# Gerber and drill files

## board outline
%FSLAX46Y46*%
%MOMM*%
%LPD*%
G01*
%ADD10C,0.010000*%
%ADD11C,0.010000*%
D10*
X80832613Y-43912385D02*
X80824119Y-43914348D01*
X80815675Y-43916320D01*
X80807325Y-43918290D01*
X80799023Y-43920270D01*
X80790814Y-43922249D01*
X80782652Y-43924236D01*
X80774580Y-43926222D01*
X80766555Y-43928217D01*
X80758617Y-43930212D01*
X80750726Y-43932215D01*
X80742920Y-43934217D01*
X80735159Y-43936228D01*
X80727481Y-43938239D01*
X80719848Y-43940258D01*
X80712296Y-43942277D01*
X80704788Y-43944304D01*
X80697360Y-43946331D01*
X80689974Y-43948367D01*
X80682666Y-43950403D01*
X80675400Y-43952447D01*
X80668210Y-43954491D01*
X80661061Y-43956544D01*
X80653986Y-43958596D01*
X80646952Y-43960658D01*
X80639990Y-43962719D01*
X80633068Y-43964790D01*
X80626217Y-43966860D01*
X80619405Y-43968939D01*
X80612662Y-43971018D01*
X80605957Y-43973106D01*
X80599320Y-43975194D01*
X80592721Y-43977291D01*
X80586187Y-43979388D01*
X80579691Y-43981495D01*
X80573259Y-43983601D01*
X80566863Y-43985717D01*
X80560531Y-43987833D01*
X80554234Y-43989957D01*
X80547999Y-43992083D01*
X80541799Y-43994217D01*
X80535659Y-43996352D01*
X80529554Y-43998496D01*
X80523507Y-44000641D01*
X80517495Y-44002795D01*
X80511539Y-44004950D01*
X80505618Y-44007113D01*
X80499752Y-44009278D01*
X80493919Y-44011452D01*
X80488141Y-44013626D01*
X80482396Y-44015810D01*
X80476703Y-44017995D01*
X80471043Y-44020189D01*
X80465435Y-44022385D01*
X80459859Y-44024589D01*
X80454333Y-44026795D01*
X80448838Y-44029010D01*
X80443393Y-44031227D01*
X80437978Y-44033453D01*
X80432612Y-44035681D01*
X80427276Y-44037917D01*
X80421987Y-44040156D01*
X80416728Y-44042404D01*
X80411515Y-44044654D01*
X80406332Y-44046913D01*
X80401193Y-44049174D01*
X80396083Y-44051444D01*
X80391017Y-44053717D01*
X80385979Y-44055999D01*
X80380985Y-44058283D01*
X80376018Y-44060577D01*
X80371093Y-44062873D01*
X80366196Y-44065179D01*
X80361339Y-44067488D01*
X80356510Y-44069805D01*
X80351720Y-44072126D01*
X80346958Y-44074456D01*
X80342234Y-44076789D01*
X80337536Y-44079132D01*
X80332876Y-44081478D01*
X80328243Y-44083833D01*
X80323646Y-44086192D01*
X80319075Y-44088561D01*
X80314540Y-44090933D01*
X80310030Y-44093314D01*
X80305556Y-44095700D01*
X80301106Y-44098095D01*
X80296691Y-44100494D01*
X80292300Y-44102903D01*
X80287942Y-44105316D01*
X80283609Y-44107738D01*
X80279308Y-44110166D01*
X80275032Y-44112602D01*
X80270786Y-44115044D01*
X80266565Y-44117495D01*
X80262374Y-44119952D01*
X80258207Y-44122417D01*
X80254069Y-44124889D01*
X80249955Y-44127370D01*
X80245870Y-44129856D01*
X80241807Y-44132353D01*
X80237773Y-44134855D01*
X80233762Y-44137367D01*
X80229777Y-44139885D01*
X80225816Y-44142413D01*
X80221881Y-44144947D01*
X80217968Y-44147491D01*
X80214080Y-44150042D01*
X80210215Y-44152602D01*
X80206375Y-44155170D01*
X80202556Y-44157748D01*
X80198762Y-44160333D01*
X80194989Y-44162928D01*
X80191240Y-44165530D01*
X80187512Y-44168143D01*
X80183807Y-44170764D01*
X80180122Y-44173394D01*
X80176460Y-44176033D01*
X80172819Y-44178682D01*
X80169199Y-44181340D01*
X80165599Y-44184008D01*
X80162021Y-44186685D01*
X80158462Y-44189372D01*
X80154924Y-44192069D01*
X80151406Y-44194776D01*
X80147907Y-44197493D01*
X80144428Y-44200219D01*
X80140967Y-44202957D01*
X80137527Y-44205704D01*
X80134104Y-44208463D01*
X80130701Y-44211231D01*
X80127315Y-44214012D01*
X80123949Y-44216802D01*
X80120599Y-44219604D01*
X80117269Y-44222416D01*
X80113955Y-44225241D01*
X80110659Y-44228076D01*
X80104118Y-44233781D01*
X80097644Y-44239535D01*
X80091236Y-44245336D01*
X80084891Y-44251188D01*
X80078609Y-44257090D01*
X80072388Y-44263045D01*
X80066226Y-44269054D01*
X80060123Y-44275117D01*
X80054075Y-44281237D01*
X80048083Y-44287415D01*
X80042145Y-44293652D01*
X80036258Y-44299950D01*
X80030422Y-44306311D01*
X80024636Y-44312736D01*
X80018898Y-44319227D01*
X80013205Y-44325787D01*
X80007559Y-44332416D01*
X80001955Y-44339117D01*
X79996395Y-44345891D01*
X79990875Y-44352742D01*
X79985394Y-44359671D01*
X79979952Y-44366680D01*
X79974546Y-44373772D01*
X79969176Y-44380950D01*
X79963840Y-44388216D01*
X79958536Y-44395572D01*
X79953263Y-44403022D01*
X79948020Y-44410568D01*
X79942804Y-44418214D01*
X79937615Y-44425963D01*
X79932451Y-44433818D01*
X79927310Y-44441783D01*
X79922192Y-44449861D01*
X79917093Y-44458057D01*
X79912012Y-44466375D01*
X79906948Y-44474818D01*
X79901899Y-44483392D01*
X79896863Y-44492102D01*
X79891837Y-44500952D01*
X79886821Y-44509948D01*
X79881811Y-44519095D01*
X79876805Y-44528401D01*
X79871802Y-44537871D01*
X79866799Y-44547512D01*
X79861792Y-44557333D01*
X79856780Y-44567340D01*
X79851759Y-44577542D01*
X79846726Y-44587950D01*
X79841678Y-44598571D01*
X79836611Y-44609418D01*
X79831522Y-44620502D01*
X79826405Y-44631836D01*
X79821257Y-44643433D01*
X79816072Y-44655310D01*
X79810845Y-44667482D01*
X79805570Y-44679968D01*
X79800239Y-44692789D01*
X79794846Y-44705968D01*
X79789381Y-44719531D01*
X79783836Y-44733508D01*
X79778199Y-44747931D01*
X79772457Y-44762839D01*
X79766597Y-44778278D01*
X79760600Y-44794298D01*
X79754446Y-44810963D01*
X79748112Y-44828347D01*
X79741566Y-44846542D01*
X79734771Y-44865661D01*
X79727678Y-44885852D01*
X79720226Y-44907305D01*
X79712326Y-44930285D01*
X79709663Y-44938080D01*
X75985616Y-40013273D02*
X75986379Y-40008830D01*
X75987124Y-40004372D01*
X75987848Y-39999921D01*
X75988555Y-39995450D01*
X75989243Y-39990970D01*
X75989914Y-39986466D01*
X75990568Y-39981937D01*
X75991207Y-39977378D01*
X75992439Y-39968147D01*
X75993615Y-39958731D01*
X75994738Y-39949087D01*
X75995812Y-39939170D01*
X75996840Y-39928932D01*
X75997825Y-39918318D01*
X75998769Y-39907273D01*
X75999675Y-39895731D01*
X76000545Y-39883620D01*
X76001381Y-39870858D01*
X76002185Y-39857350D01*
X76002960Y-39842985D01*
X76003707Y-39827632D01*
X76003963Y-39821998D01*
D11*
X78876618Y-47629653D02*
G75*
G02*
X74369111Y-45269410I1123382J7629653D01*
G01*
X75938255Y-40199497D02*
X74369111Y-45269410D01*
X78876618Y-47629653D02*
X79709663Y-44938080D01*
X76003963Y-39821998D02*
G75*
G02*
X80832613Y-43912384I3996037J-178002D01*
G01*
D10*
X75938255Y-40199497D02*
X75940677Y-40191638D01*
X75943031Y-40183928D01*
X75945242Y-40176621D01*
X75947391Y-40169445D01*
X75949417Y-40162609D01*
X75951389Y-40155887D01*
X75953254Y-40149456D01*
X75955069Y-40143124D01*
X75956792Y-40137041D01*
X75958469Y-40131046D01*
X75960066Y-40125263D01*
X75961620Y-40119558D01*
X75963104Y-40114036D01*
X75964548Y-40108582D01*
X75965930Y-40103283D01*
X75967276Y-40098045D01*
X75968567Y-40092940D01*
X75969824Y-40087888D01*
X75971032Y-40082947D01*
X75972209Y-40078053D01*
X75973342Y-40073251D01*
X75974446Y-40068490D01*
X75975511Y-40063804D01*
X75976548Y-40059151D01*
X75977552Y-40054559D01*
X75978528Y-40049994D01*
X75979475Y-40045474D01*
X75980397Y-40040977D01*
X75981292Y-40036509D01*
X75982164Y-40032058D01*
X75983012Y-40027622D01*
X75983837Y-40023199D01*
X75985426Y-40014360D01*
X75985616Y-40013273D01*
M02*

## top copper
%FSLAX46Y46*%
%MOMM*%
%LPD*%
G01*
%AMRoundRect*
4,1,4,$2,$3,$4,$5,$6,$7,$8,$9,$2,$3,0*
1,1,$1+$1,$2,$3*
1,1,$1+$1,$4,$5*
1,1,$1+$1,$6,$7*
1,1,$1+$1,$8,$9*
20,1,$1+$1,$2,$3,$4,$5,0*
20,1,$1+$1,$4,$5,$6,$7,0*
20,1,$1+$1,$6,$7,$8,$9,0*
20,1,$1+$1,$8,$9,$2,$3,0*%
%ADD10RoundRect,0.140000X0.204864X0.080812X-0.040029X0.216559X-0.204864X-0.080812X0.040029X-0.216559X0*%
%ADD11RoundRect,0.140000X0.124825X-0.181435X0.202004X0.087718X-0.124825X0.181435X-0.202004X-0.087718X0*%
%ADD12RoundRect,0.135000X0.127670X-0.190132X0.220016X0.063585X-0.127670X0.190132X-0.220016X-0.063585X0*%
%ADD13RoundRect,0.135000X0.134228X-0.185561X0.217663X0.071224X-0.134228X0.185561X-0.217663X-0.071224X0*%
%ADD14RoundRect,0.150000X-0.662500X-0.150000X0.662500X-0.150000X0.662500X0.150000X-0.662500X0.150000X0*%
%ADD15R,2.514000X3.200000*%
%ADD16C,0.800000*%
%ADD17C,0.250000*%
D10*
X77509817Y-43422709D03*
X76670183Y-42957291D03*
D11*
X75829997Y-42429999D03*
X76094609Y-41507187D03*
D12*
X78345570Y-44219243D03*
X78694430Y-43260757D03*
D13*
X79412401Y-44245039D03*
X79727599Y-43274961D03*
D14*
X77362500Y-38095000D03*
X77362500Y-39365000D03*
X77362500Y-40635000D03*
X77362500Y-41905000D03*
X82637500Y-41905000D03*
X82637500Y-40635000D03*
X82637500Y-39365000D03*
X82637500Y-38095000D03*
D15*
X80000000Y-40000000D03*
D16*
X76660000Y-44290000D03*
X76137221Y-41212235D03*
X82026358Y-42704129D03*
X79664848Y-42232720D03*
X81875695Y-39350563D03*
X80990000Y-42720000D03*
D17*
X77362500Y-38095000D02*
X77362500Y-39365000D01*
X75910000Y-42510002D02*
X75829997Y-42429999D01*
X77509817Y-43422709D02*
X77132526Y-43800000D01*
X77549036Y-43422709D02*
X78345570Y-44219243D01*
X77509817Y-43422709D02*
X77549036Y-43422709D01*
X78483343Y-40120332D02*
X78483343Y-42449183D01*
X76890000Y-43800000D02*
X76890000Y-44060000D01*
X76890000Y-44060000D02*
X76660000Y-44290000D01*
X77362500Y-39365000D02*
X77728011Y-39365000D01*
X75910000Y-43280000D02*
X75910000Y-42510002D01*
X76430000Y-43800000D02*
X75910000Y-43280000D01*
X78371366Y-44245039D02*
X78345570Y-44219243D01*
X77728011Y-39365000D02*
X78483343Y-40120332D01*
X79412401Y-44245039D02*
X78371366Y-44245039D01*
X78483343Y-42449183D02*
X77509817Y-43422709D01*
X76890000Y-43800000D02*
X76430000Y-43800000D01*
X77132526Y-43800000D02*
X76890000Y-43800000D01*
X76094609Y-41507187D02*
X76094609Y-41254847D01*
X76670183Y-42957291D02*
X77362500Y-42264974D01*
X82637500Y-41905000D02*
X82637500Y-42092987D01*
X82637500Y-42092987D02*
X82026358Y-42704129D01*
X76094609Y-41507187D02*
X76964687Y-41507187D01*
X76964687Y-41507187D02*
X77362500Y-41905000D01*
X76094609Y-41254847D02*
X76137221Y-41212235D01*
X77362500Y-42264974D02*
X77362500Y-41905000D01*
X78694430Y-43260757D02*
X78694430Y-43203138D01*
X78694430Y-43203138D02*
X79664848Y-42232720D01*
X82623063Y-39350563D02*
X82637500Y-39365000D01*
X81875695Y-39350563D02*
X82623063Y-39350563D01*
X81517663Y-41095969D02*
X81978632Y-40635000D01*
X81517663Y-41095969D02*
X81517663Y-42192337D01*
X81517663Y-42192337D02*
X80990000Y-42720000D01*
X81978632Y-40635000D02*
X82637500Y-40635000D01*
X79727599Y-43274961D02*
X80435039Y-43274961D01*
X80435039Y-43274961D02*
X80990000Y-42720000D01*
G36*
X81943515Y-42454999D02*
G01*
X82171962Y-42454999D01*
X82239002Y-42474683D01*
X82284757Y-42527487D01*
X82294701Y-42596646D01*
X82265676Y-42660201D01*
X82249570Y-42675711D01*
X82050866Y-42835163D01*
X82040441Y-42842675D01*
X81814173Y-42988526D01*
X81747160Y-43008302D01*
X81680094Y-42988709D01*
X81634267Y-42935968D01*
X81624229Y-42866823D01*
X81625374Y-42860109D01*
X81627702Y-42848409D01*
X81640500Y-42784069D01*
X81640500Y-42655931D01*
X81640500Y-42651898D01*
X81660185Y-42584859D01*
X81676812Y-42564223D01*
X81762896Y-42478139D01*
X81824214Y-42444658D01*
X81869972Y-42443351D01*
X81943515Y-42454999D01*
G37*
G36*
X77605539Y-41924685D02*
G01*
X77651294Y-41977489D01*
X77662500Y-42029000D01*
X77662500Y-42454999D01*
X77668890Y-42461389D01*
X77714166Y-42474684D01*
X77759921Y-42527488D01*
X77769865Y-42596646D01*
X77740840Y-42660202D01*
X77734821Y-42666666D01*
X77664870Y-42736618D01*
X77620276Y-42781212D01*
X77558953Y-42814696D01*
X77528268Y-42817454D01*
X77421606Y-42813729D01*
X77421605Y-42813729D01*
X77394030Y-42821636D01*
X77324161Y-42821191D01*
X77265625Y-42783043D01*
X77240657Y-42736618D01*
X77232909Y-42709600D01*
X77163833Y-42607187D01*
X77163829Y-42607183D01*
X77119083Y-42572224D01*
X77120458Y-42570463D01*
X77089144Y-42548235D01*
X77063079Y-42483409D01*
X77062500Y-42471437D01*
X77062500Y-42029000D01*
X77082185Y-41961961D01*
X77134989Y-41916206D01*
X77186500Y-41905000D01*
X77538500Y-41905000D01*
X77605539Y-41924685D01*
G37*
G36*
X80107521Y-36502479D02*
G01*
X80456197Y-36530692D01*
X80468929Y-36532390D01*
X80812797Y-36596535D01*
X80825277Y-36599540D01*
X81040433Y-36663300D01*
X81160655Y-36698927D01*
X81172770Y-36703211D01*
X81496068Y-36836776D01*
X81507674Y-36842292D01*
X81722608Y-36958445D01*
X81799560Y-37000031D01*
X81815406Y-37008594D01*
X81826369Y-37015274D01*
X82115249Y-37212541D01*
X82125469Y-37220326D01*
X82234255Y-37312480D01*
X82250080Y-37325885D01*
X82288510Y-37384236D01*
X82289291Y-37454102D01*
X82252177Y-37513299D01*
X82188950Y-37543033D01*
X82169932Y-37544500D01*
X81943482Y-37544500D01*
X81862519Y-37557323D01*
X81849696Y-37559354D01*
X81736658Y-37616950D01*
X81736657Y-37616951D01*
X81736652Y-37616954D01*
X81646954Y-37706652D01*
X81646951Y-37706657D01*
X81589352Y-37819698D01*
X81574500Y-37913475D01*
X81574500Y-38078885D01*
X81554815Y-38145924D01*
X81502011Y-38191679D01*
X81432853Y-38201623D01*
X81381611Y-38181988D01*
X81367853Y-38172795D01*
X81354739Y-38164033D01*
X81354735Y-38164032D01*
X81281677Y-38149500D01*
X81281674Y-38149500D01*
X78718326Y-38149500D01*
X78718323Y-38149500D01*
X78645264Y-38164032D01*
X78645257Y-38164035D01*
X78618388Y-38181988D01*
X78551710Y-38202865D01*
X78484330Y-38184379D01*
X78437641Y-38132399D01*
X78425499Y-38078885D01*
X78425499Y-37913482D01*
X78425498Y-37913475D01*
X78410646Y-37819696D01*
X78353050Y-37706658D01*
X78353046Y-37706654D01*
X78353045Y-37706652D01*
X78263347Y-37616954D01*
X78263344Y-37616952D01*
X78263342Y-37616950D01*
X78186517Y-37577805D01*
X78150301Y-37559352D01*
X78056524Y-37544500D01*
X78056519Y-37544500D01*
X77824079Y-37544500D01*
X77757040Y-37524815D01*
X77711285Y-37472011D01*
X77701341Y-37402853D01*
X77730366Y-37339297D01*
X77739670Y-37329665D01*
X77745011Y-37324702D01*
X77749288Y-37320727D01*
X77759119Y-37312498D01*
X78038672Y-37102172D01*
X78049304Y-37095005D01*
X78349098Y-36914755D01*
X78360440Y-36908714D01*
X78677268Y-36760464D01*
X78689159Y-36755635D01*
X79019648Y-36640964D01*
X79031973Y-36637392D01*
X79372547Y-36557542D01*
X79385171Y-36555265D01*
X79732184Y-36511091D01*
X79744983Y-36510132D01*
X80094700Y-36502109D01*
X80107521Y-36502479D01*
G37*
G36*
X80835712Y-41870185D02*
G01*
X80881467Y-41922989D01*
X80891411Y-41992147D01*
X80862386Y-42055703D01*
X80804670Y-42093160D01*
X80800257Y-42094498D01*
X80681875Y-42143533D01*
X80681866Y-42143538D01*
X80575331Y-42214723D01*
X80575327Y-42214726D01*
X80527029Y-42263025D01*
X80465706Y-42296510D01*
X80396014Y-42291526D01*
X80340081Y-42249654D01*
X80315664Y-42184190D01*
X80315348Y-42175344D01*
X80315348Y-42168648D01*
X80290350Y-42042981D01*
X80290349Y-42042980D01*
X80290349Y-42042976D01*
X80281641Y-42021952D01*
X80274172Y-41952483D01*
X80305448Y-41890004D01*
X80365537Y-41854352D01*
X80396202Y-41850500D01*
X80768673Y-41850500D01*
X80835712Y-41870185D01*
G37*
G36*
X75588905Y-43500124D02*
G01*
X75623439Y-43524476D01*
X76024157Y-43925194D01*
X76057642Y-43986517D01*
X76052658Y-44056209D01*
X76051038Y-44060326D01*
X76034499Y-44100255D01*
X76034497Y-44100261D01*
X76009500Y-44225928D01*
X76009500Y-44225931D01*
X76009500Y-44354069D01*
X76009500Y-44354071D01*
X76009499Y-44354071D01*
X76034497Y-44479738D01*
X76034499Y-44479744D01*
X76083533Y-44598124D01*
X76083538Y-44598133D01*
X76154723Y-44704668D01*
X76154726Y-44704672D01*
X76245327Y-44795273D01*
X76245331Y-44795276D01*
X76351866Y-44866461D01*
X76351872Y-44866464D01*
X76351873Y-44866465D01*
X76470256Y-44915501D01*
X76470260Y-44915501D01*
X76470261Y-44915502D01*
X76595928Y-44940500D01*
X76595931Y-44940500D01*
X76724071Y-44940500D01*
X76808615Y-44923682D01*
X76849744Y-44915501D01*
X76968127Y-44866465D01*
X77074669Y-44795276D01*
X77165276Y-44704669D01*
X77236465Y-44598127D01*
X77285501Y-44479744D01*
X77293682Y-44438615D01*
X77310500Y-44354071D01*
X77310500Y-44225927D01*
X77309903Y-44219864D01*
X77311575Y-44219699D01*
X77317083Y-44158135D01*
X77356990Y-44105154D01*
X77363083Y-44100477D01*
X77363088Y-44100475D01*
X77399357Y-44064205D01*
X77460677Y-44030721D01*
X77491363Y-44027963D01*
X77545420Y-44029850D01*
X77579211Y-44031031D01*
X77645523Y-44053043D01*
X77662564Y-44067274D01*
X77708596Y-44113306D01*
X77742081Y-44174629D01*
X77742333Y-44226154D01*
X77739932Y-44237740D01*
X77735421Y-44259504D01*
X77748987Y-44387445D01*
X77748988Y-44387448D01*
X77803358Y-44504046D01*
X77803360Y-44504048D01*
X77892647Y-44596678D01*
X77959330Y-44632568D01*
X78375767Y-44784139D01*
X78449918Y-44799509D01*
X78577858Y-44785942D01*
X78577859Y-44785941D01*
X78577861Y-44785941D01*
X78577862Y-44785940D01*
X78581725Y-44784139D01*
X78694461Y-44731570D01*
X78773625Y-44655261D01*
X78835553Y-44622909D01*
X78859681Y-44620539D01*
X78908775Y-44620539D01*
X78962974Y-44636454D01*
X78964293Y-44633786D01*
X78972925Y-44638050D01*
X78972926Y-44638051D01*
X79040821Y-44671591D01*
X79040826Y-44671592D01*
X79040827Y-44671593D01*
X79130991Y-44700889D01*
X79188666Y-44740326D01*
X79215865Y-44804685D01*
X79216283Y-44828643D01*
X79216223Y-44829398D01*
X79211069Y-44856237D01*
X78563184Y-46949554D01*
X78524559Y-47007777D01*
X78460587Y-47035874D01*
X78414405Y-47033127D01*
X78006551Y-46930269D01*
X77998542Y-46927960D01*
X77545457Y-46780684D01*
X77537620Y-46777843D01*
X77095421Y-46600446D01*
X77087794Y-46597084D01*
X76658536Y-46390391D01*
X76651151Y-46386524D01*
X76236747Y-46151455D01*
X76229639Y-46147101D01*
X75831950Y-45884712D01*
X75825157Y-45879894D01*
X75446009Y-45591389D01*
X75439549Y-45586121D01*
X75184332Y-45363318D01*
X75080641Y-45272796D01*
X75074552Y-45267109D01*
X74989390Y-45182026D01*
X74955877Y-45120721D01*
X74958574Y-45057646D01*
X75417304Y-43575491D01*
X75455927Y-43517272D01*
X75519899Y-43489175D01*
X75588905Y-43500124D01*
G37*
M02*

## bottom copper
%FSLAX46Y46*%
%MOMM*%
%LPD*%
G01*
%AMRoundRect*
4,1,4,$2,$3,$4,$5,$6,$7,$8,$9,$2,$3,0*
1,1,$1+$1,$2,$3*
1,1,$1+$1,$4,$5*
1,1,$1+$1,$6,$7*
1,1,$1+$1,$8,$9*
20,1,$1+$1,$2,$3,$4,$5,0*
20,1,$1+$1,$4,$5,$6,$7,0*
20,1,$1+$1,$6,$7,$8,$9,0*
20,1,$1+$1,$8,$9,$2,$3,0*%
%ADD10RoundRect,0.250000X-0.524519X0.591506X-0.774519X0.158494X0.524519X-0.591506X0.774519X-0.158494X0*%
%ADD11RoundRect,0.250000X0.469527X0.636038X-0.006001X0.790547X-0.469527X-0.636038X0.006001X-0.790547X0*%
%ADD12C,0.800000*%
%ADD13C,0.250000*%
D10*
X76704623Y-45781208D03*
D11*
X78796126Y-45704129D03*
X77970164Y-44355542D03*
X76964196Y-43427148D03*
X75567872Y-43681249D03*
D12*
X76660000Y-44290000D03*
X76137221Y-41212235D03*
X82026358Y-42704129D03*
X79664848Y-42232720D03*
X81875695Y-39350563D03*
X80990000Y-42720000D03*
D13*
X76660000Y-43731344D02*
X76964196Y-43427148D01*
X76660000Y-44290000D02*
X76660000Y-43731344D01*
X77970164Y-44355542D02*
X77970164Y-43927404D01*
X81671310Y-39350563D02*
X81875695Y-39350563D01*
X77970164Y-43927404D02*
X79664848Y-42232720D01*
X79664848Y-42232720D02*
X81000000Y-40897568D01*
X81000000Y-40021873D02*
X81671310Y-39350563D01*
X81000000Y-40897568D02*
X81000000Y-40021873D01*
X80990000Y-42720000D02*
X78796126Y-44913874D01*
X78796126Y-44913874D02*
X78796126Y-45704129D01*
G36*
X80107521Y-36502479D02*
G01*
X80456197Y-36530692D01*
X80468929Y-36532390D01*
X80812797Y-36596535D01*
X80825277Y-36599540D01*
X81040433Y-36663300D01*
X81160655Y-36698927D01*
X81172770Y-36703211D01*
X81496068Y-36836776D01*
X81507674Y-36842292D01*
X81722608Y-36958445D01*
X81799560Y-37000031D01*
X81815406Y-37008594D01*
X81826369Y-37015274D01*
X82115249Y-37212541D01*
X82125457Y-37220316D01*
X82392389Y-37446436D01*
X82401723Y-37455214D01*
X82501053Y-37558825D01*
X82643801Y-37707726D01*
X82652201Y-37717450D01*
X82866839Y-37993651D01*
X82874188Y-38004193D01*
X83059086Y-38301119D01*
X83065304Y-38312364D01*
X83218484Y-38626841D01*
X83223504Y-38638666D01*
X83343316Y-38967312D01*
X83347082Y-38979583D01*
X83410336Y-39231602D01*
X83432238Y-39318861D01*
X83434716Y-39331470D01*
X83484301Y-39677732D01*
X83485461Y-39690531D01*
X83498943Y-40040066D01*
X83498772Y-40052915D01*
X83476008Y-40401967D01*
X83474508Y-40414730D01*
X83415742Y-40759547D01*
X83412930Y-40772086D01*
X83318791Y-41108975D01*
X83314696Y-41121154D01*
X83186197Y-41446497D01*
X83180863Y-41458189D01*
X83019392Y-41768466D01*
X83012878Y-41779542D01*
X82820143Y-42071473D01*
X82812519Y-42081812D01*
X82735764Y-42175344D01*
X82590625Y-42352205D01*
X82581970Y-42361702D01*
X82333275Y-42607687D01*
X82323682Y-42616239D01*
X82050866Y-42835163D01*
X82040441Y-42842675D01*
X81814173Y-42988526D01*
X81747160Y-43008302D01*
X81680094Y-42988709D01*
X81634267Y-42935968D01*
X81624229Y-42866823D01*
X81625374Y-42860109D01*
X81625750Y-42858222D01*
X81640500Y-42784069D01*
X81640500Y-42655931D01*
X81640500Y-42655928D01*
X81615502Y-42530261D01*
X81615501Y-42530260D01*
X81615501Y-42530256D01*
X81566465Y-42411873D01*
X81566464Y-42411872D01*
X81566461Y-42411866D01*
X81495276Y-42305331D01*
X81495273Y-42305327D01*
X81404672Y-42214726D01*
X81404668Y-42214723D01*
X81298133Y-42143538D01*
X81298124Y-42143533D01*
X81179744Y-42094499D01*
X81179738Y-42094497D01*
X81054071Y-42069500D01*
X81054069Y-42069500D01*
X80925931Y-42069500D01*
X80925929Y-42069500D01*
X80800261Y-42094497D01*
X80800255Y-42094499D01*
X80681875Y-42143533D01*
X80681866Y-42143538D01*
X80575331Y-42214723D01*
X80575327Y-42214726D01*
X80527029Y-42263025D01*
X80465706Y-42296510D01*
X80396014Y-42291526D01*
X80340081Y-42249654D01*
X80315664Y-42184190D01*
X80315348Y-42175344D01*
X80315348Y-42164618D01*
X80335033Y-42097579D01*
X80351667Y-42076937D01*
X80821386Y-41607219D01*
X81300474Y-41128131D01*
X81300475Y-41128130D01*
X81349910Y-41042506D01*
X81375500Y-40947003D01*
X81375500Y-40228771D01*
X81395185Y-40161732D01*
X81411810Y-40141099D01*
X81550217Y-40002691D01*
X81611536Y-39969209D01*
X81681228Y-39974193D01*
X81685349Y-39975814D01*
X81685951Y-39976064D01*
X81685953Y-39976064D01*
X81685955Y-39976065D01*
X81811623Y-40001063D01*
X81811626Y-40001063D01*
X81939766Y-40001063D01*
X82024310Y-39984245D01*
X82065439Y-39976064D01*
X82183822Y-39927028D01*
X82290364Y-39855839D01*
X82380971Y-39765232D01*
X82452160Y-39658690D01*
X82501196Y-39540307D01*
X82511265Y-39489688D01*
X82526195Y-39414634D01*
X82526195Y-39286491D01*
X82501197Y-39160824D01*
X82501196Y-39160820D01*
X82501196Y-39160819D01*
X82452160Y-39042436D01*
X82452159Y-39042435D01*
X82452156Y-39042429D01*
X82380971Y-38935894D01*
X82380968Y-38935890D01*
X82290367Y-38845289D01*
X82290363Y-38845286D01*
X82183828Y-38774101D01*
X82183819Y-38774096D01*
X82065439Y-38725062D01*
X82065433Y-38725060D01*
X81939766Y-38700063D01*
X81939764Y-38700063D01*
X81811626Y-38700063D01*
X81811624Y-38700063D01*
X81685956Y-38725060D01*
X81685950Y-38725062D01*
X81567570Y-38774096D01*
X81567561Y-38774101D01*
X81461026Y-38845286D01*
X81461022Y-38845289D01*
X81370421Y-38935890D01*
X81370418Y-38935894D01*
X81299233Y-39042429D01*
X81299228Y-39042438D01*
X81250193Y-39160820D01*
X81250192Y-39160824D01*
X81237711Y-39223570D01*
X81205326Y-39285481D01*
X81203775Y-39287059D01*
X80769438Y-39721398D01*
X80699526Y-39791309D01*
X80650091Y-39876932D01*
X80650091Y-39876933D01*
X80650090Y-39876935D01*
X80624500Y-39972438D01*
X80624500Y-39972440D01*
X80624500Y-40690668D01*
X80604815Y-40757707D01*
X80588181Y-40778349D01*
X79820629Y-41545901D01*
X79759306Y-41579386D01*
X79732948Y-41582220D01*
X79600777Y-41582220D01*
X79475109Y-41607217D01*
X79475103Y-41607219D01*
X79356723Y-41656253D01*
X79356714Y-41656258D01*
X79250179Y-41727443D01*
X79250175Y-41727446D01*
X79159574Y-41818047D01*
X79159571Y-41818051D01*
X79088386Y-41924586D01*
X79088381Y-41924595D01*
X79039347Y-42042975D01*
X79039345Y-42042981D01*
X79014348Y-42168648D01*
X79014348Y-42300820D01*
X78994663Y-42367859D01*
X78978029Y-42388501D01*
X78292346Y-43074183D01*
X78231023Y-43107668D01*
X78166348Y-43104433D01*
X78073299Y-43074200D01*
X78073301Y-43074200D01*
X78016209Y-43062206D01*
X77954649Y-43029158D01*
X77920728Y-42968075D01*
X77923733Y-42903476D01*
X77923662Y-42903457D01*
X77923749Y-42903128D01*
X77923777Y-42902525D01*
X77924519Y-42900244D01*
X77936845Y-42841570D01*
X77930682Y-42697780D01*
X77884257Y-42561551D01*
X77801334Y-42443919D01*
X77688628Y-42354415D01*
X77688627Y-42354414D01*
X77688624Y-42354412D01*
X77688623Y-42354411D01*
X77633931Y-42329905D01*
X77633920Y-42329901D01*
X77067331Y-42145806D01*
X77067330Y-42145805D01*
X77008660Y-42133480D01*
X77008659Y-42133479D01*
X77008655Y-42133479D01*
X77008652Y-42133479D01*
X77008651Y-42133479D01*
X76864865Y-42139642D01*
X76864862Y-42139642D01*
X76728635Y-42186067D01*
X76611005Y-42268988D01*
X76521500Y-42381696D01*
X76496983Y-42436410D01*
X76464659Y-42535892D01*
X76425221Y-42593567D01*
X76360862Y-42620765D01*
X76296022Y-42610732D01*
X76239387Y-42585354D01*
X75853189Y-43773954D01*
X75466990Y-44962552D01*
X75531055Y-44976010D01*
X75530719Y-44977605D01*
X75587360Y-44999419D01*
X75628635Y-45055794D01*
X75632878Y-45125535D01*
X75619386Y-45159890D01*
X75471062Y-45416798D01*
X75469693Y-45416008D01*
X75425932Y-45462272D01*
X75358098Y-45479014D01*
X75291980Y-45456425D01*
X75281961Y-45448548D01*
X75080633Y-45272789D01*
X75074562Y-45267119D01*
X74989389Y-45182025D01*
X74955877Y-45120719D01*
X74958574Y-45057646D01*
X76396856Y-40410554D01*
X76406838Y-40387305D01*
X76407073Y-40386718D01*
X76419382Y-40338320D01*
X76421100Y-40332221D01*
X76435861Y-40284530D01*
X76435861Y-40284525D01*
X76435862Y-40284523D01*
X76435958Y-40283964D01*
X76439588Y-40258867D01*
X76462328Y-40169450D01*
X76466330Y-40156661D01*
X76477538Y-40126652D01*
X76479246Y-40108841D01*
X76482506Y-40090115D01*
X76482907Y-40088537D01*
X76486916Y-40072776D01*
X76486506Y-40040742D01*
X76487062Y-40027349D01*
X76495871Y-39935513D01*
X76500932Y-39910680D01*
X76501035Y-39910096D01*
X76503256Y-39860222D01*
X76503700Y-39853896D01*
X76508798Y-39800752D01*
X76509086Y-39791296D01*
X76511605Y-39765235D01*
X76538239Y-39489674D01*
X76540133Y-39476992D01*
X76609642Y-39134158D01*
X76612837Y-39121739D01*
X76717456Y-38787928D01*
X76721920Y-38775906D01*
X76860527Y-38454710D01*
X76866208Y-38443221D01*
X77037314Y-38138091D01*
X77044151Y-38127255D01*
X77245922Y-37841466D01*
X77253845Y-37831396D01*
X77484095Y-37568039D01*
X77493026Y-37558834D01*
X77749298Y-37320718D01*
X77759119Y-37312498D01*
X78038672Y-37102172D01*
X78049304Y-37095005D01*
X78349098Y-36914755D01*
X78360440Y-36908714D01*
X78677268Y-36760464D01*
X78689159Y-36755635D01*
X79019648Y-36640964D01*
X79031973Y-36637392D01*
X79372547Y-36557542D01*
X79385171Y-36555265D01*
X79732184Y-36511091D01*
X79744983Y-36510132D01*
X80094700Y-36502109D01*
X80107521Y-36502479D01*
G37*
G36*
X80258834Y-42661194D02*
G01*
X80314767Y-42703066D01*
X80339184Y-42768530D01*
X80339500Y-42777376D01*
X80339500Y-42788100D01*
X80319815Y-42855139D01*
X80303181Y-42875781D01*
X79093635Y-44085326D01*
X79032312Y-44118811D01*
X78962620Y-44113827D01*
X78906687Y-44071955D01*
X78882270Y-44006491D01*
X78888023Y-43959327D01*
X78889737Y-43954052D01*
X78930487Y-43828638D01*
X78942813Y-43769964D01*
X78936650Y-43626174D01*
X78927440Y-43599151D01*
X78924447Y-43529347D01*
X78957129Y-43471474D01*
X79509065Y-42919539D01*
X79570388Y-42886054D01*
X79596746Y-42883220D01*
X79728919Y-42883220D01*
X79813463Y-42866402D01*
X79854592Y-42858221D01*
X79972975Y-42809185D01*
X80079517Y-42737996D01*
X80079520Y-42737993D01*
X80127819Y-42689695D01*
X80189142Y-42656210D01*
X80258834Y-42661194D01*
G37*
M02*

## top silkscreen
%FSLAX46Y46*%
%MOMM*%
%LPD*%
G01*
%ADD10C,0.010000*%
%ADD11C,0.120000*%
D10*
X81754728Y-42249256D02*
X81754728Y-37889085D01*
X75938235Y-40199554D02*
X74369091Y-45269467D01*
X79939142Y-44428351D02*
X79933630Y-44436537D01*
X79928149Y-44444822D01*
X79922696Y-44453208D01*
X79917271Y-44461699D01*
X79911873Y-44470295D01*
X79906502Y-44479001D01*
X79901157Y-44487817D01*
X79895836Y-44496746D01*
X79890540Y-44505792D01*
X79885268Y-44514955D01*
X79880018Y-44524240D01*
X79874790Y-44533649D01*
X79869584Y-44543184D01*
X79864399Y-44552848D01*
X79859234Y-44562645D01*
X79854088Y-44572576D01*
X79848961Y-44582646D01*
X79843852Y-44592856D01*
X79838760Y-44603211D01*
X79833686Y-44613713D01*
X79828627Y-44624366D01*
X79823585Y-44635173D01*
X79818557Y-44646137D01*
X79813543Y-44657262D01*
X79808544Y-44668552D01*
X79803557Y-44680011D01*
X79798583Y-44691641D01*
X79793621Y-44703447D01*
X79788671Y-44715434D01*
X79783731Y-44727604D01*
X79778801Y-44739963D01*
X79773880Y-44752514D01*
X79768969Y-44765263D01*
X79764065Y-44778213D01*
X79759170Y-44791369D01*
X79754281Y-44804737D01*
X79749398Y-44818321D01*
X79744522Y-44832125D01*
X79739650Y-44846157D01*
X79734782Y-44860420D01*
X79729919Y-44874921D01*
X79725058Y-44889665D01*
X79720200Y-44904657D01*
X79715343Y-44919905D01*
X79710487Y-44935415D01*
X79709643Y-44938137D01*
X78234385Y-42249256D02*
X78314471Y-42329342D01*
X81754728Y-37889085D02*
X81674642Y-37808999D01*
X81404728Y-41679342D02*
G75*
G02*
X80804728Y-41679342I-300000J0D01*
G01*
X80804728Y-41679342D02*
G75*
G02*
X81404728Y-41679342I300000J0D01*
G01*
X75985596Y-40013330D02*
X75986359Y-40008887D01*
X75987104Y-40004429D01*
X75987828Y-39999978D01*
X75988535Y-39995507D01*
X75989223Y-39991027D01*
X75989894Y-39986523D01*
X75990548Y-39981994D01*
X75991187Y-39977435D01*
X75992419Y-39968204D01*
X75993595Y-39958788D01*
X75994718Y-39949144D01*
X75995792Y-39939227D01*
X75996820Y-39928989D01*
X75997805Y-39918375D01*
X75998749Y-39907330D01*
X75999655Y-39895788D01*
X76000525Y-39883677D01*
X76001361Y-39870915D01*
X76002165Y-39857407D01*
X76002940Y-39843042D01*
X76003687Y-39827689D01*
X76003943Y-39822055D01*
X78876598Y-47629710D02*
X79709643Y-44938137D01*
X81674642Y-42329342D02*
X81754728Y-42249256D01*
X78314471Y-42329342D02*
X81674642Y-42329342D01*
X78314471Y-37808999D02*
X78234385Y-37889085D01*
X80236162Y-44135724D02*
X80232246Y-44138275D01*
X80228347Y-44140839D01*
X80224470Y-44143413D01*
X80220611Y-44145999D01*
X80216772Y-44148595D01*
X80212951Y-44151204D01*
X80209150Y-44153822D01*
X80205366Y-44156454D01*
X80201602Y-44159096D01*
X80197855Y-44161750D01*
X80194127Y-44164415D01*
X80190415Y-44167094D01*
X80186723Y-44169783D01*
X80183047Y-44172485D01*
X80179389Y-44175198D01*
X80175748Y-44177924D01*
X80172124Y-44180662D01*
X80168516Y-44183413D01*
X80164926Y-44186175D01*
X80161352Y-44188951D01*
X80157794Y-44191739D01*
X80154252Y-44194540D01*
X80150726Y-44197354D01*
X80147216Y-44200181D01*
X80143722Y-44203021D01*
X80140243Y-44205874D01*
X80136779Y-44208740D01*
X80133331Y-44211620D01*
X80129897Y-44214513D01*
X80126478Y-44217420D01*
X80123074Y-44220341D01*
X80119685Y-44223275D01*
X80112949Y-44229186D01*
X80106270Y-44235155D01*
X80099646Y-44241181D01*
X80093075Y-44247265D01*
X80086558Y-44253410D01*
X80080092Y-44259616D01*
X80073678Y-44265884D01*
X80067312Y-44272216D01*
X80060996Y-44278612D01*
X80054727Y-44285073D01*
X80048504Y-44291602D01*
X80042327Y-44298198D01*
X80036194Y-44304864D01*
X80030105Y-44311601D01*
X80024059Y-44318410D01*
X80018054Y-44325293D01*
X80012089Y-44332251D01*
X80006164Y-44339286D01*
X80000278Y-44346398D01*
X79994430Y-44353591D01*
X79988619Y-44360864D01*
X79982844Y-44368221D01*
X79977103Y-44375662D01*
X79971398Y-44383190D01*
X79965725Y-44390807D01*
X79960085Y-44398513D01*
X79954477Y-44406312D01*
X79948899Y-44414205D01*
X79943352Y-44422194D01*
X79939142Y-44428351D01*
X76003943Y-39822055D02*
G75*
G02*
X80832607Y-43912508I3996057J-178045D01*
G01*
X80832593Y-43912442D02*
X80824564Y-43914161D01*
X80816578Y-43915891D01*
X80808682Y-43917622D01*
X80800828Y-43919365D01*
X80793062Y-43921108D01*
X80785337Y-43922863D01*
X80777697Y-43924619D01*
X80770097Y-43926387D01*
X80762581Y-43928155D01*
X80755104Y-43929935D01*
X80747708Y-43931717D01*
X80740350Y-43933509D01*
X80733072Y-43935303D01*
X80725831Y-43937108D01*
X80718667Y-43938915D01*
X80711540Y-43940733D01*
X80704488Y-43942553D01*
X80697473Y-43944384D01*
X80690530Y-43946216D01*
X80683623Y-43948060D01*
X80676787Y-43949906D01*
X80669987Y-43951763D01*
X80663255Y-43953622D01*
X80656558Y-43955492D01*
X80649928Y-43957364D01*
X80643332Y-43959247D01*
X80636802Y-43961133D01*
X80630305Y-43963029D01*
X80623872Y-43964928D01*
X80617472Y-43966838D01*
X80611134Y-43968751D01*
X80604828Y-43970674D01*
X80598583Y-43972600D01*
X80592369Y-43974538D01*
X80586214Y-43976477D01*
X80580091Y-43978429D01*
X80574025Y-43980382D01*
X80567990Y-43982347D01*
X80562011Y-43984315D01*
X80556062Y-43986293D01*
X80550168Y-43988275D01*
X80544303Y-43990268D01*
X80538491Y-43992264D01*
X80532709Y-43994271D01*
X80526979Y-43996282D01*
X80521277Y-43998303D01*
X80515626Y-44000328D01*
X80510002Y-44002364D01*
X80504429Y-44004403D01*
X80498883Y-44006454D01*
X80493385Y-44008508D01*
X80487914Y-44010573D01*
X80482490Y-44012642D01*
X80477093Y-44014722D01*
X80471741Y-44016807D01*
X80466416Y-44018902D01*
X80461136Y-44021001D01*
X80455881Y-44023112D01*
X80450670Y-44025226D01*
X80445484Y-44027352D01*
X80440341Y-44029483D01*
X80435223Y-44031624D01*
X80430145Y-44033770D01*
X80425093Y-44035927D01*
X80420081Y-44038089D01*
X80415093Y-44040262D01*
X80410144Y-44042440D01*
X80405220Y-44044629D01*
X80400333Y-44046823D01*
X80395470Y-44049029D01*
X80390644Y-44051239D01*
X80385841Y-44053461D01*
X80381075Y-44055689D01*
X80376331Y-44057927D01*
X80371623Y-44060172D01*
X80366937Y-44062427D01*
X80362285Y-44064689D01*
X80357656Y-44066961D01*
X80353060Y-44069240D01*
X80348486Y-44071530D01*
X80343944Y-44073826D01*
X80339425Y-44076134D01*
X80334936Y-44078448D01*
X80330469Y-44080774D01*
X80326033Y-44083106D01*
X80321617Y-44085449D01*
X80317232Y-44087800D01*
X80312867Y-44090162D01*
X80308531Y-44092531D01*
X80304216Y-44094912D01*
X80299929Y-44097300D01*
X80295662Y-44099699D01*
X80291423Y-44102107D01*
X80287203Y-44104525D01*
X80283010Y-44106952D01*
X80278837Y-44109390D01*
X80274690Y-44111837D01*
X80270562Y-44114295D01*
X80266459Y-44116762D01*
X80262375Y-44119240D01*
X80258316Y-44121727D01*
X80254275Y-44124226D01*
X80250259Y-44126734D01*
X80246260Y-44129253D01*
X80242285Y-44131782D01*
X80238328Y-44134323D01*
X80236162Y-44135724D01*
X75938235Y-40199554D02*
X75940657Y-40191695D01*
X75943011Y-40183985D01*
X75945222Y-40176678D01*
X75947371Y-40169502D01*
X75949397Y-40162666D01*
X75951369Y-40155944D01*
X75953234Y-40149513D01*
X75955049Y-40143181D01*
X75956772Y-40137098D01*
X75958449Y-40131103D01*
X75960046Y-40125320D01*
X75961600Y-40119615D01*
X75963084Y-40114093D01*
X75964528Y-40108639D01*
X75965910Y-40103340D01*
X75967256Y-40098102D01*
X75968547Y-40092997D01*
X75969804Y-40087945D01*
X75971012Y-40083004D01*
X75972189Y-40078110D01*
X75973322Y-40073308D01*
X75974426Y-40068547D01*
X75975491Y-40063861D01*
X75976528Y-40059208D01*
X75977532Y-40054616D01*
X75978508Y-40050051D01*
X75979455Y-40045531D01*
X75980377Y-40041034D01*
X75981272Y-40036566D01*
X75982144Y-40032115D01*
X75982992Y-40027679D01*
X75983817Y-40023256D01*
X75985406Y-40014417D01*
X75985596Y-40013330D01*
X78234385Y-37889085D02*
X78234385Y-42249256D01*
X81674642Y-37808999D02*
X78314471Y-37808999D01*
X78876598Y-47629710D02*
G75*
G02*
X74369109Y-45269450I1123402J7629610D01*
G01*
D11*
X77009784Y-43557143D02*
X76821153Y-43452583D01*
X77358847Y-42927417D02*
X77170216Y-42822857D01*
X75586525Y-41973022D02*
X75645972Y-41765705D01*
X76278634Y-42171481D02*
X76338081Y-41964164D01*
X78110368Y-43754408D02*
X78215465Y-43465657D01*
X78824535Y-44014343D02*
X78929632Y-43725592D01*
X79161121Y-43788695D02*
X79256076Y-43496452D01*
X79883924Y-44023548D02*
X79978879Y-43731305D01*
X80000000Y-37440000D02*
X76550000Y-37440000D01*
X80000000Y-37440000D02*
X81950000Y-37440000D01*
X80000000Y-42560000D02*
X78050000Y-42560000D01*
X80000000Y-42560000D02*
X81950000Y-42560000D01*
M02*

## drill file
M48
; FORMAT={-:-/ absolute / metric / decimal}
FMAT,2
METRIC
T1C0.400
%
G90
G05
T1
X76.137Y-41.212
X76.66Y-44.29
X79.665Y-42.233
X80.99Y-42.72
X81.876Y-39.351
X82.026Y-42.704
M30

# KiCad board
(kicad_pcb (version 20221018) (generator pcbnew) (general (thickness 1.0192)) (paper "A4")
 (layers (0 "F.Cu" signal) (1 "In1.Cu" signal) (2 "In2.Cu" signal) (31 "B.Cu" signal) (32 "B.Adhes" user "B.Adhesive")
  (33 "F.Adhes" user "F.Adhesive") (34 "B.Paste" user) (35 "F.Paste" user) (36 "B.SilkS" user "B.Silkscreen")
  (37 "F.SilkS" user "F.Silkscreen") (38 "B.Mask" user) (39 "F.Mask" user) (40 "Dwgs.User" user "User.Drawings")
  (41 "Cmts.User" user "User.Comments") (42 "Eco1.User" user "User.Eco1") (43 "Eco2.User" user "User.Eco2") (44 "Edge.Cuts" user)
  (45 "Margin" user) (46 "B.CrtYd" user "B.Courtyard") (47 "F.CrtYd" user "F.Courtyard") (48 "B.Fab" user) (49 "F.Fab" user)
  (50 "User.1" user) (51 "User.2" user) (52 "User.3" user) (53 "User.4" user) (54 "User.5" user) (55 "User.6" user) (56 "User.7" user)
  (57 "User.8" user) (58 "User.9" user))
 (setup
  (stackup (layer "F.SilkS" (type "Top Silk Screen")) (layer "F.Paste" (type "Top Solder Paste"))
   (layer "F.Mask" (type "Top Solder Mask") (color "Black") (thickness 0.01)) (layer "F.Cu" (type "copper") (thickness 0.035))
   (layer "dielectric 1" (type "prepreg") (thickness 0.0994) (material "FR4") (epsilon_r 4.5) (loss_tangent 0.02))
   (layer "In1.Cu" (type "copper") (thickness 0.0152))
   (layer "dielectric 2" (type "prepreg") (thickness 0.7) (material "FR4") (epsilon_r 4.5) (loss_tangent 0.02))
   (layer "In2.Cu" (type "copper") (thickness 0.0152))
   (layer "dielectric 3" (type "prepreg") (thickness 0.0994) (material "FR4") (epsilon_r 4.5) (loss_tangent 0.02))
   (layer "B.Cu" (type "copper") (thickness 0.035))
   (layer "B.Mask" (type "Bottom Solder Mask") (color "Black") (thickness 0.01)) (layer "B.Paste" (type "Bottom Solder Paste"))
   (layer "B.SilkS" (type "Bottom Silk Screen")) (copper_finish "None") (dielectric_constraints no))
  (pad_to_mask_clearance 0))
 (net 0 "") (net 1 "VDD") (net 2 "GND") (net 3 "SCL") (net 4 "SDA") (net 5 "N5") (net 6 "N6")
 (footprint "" (layer "F.Cu") (at 76.704623 45.781208 78)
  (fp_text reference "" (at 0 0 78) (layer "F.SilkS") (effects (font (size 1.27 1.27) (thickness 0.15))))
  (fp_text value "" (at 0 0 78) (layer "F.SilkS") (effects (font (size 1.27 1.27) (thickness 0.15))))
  (pad "9" smd roundrect (at 0 0 240) (size 1 2) (layers "B.Cu" "B.Mask") (roundrect_rratio 0.25)))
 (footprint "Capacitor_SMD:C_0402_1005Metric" (layer "F.Cu") (at 77.09 43.19 151)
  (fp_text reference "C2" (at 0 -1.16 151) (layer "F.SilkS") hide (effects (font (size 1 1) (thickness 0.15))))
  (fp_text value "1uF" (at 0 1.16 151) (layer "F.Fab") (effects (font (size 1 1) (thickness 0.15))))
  (fp_line (start -0.107836 -0.36) (end 0.107836 -0.36) (stroke (width 0.12) (type solid)) (layer "F.SilkS"))
  (fp_line (start -0.107836 0.36) (end 0.107836 0.36) (stroke (width 0.12) (type solid)) (layer "F.SilkS"))
  (pad "1" smd roundrect (at -0.48 0 151) (size 0.56 0.62) (layers "F.Cu" "F.Paste" "F.Mask") (roundrect_rratio 0.25) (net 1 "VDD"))
  (pad "2" smd roundrect (at 0.48 0 151) (size 0.56 0.62) (layers "F.Cu" "F.Paste" "F.Mask") (roundrect_rratio 0.25) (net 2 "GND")))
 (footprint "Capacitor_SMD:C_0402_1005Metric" (layer "F.Cu") (at 75.962303 41.968593 74)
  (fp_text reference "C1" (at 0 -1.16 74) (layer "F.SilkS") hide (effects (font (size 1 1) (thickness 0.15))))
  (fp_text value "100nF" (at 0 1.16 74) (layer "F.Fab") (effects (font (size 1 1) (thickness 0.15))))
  (fp_line (start -0.107836 -0.36) (end 0.107836 -0.36) (stroke (width 0.12) (type solid)) (layer "F.SilkS"))
  (fp_line (start -0.107836 0.36) (end 0.107836 0.36) (stroke (width 0.12) (type solid)) (layer "F.SilkS"))
  (pad "1" smd roundrect (at -0.48 0 74) (size 0.56 0.62) (layers "F.Cu" "F.Paste" "F.Mask") (roundrect_rratio 0.25) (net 1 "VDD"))
  (pad "2" smd roundrect (at 0.48 0 74) (size 0.56 0.62) (layers "F.Cu" "F.Paste" "F.Mask") (roundrect_rratio 0.25) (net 2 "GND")))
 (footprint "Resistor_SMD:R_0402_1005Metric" (layer "F.Cu") (at 78.52 43.74 70)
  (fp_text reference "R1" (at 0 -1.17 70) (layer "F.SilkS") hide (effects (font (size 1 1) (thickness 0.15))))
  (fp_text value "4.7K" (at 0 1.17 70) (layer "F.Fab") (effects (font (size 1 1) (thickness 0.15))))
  (fp_line (start -0.153641 -0.38) (end 0.153641 -0.38) (stroke (width 0.12) (type solid)) (layer "F.SilkS"))
  (fp_line (start -0.153641 0.38) (end 0.153641 0.38) (stroke (width 0.12) (type solid)) (layer "F.SilkS"))
  (pad "1" smd roundrect (at -0.51 0 70) (size 0.54 0.64) (layers "F.Cu" "F.Paste" "F.Mask") (roundrect_rratio 0.25) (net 1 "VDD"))
  (pad "2" smd roundrect (at 0.51 0 70) (size 0.54 0.64) (layers "F.Cu" "F.Paste" "F.Mask") (roundrect_rratio 0.25) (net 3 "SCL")))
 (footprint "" (layer "F.Cu") (at 78.796126 45.704129)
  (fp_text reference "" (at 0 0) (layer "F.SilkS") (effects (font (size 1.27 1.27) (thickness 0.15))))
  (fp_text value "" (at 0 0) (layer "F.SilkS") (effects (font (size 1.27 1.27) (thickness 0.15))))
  (pad "9" smd roundrect (at 0 0 162) (size 1 2) (layers "B.Cu" "B.Mask") (roundrect_rratio 0.25) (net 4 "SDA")))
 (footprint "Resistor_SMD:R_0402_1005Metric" (layer "F.Cu") (at 79.57 43.76 72)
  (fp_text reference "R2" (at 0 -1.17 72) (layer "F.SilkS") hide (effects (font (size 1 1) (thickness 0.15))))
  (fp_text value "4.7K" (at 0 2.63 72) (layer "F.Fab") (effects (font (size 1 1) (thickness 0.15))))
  (fp_line (start -0.153641 -0.38) (end 0.153641 -0.38) (stroke (width 0.12) (type solid)) (layer "F.SilkS"))
  (fp_line (start -0.153641 0.38) (end 0.153641 0.38) (stroke (width 0.12) (type solid)) (layer "F.SilkS"))
  (pad "1" smd roundrect (at -0.51 0 72) (size 0.54 0.64) (layers "F.Cu" "F.Paste" "F.Mask") (roundrect_rratio 0.25) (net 1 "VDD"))
  (pad "2" smd roundrect (at 0.51 0 72) (size 0.54 0.64) (layers "F.Cu" "F.Paste" "F.Mask") (roundrect_rratio 0.25) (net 4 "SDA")))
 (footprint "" (layer "F.Cu") (at 77.970164 44.355542)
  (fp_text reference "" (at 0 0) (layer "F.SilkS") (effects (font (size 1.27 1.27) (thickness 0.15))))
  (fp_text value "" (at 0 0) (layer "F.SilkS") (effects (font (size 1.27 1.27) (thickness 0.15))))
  (pad "9" smd roundrect (at 0 0 162) (size 1 2) (layers "B.Cu" "B.Mask") (roundrect_rratio 0.25) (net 3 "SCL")))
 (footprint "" (layer "F.Cu") (at 76.964196 43.427148)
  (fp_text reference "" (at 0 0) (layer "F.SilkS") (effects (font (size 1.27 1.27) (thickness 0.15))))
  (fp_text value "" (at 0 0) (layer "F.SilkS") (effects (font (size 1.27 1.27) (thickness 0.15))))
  (pad "9" smd roundrect (at 0 0 162) (size 1 2) (layers "B.Cu" "B.Mask") (roundrect_rratio 0.25) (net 1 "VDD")))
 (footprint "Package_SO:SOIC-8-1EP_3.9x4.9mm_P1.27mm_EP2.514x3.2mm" (layer "F.Cu") (at 80 40)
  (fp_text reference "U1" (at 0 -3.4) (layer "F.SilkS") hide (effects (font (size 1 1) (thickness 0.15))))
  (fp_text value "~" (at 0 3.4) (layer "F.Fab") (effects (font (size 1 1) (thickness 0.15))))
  (fp_line (start 0 -2.56) (end -3.45 -2.56) (stroke (width 0.12) (type solid)) (layer "F.SilkS"))
  (fp_line (start 0 -2.56) (end 1.95 -2.56) (stroke (width 0.12) (type solid)) (layer "F.SilkS"))
  (fp_line (start 0 2.56) (end -1.95 2.56) (stroke (width 0.12) (type solid)) (layer "F.SilkS"))
  (fp_line (start 0 2.56) (end 1.95 2.56) (stroke (width 0.12) (type solid)) (layer "F.SilkS"))
  (pad "" smd roundrect (at -0.63 -0.8) (size 1.01 1.29) (layers "F.Paste") (roundrect_rratio 0.2475247525))
  (pad "" smd roundrect (at -0.63 0.8) (size 1.01 1.29) (layers "F.Paste") (roundrect_rratio 0.2475247525))
  (pad "" smd roundrect (at 0.63 -0.8) (size 1.01 1.29) (layers "F.Paste") (roundrect_rratio 0.2475247525))
  (pad "" smd roundrect (at 0.63 0.8) (size 1.01 1.29) (layers "F.Paste") (roundrect_rratio 0.2475247525))
  (pad "1" smd roundrect (at -2.6375 -1.905) (size 1.625 0.6) (layers "F.Cu" "F.Paste" "F.Mask") (roundrect_rratio 0.25) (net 1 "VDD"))
  (pad "2" smd roundrect (at -2.6375 -0.635) (size 1.625 0.6) (layers "F.Cu" "F.Paste" "F.Mask") (roundrect_rratio 0.25) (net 1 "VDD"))
  (pad "3" smd roundrect (at -2.6375 0.635) (size 1.625 0.6) (layers "F.Cu" "F.Paste" "F.Mask") (roundrect_rratio 0.25) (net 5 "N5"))
  (pad "4" smd roundrect (at -2.6375 1.905) (size 1.625 0.6) (layers "F.Cu" "F.Paste" "F.Mask") (roundrect_rratio 0.25) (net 2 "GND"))
  (pad "5" smd roundrect (at 2.6375 1.905) (size 1.625 0.6) (layers "F.Cu" "F.Paste" "F.Mask") (roundrect_rratio 0.25) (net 2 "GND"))
  (pad "6" smd roundrect (at 2.6375 0.635) (size 1.625 0.6) (layers "F.Cu" "F.Paste" "F.Mask") (roundrect_rratio 0.25) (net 4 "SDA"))
  (pad "7" smd roundrect (at 2.6375 -0.635) (size 1.625 0.6) (layers "F.Cu" "F.Paste" "F.Mask") (roundrect_rratio 0.25) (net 3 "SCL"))
  (pad "8" smd roundrect (at 2.6375 -1.905) (size 1.625 0.6) (layers "F.Cu" "F.Paste" "F.Mask") (roundrect_rratio 0.25) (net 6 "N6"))
  (pad "9" smd rect (at 0 0) (size 2.514 3.2) (layers "F.Cu" "F.Mask")))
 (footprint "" (layer "B.Cu") (at 75.567872 43.681249 162)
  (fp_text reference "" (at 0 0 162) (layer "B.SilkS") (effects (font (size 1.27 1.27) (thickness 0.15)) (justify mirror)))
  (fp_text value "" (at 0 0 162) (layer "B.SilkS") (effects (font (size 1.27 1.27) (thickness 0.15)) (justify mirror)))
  (pad "9" smd roundrect (at 0 0 162) (size 1 2) (layers "B.Cu" "B.Mask") (roundrect_rratio 0.25) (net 2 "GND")))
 (gr_line (start 81.754728 42.249256) (end 81.754728 37.889085) (stroke (width 0.01) (type solid)) (layer "F.SilkS"))
 (gr_line (start 75.938235 40.199554) (end 74.369091 45.269467) (stroke (width 0.01) (type solid)) (layer "F.SilkS"))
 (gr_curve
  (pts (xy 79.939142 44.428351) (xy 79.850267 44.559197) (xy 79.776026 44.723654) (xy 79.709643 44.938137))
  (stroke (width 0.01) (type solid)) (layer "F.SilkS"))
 (gr_line (start 78.234385 42.249256) (end 78.314471 42.329342) (stroke (width 0.01) (type solid)) (layer "F.SilkS"))
 (gr_line (start 81.754728 37.889085) (end 81.674642 37.808999) (stroke (width 0.01) (type solid)) (layer "F.SilkS"))
 (gr_circle (center 81.104728 41.679342) (end 81.404728 41.679342) (stroke (width 0.01) (type solid)) (fill none) (layer "F.SilkS"))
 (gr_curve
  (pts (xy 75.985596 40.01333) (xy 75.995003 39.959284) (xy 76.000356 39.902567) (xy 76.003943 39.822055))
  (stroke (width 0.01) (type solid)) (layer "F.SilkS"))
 (gr_line (start 78.876598 47.62971) (end 79.709643 44.938137) (stroke (width 0.01) (type solid)) (layer "F.SilkS"))
 (gr_line (start 81.674642 42.329342) (end 81.754728 42.249256) (stroke (width 0.01) (type solid)) (layer "F.SilkS"))
 (gr_line (start 78.314471 42.329342) (end 81.674642 42.329342) (stroke (width 0.01) (type solid)) (layer "F.SilkS"))
 (gr_line (start 78.314471 37.808999) (end 78.234385 37.889085) (stroke (width 0.01) (type solid)) (layer "F.SilkS"))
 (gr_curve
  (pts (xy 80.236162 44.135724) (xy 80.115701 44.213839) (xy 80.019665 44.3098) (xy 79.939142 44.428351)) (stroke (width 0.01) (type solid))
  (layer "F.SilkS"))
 (gr_arc (start 76.003943 39.822055) (mid 82.585445 36.947948) (end 80.832593 43.912442) (stroke (width 0.01) (type solid))
  (layer "F.SilkS"))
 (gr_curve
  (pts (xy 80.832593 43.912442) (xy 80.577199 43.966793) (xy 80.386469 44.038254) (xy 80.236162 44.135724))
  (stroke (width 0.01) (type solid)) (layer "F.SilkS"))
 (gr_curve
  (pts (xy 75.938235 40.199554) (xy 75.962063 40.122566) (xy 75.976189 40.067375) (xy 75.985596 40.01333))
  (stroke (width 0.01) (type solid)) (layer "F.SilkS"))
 (gr_line (start 78.234385 37.889085) (end 78.234385 42.249256) (stroke (width 0.01) (type solid)) (layer "F.SilkS"))
 (gr_line (start 81.674642 37.808999) (end 78.314471 37.808999) (stroke (width 0.01) (type solid)) (layer "F.SilkS"))
 (gr_arc (start 78.876598 47.62971) (mid 76.422588 46.832031) (end 74.369091 45.269467) (stroke (width 0.01) (type solid)) (layer "F.SilkS"))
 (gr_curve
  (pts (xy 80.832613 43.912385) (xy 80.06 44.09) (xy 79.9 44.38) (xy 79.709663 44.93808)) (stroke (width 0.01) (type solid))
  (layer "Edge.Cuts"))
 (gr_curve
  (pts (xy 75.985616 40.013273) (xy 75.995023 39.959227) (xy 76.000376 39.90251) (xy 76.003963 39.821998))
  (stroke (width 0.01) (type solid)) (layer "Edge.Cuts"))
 (gr_arc (start 78.876618 47.629653) (mid 76.422608 46.831974) (end 74.369111 45.26941) (stroke (width 0.01) (type solid))
  (layer "Edge.Cuts"))
 (gr_line (start 75.938255 40.199497) (end 74.369111 45.26941) (stroke (width 0.01) (type solid)) (layer "Edge.Cuts"))
 (gr_line (start 78.876618 47.629653) (end 79.709663 44.93808) (stroke (width 0.01) (type solid)) (layer "Edge.Cuts"))
 (gr_arc (start 76.003963 39.821998) (mid 82.585465 36.947891) (end 80.832613 43.912385) (stroke (width 0.01) (type solid))
  (layer "Edge.Cuts"))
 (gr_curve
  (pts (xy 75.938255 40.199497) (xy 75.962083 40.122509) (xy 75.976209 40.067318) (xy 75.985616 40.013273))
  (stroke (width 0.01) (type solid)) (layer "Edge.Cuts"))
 (segment (start 77.3625 38.095) (end 77.3625 39.365) (width 0.25) (layer "F.Cu") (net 1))
 (segment (start 75.91 42.510002) (end 75.829997 42.429999) (width 0.25) (layer "F.Cu") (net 1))
 (segment (start 77.509817 43.422709) (end 77.132526 43.8) (width 0.25) (layer "F.Cu") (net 1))
 (segment (start 77.549036 43.422709) (end 78.34557 44.219243) (width 0.25) (layer "F.Cu") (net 1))
 (segment (start 77.509817 43.422709) (end 77.549036 43.422709) (width 0.25) (layer "F.Cu") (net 1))
 (segment (start 78.483343 40.120332) (end 78.483343 42.449183) (width 0.25) (layer "F.Cu") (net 1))
 (segment (start 76.89 43.8) (end 76.89 44.06) (width 0.25) (layer "F.Cu") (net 1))
 (segment (start 76.89 44.06) (end 76.66 44.29) (width 0.25) (layer "F.Cu") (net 1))
 (segment (start 77.3625 39.365) (end 77.728011 39.365) (width 0.25) (layer "F.Cu") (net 1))
 (segment (start 75.91 43.28) (end 75.91 42.510002) (width 0.25) (layer "F.Cu") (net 1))
 (segment (start 76.43 43.8) (end 75.91 43.28) (width 0.25) (layer "F.Cu") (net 1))
 (segment (start 78.371366 44.245039) (end 78.34557 44.219243) (width 0.25) (layer "F.Cu") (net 1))
 (segment (start 77.728011 39.365) (end 78.483343 40.120332) (width 0.25) (layer "F.Cu") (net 1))
 (segment (start 79.412401 44.245039) (end 78.371366 44.245039) (width 0.25) (layer "F.Cu") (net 1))
 (segment (start 78.483343 42.449183) (end 77.509817 43.422709) (width 0.25) (layer "F.Cu") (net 1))
 (segment (start 76.89 43.8) (end 76.43 43.8) (width 0.25) (layer "F.Cu") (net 1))
 (segment (start 77.132526 43.8) (end 76.89 43.8) (width 0.25) (layer "F.Cu") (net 1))
 (via (at 76.66 44.29) (size 0.8) (drill 0.4) (layers "F.Cu" "B.Cu") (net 1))
 (segment (start 76.66 43.731344) (end 76.964196 43.427148) (width 0.25) (layer "B.Cu") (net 1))
 (segment (start 76.66 44.29) (end 76.66 43.731344) (width 0.25) (layer "B.Cu") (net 1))
 (segment (start 76.094609 41.507187) (end 76.094609 41.254847) (width 0.25) (layer "F.Cu") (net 2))
 (segment (start 76.670183 42.957291) (end 77.3625 42.264974) (width 0.25) (layer "F.Cu") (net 2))
 (segment (start 82.6375 41.905) (end 82.6375 42.092987) (width 0.25) (layer "F.Cu") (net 2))
 (segment (start 82.6375 42.092987) (end 82.026358 42.704129) (width 0.25) (layer "F.Cu") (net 2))
 (segment (start 76.094609 41.507187) (end 76.964687 41.507187) (width 0.25) (layer "F.Cu") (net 2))
 (segment (start 76.964687 41.507187) (end 77.3625 41.905) (width 0.25) (layer "F.Cu") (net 2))
 (segment (start 76.094609 41.254847) (end 76.137221 41.212235) (width 0.25) (layer "F.Cu") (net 2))
 (segment (start 77.3625 42.264974) (end 77.3625 41.905) (width 0.25) (layer "F.Cu") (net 2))
 (via (at 76.137221 41.212235) (size 0.8) (drill 0.4) (layers "F.Cu" "B.Cu") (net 2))
 (via (at 82.026358 42.704129) (size 0.8) (drill 0.4) (layers "F.Cu" "B.Cu") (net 2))
 (segment (start 78.69443 43.260757) (end 78.69443 43.203138) (width 0.25) (layer "F.Cu") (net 3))
 (segment (start 78.69443 43.203138) (end 79.664848 42.23272) (width 0.25) (layer "F.Cu") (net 3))
 (segment (start 82.623063 39.350563) (end 82.6375 39.365) (width 0.25) (layer "F.Cu") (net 3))
 (segment (start 81.875695 39.350563) (end 82.623063 39.350563) (width 0.25) (layer "F.Cu") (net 3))
 (via (at 79.664848 42.23272) (size 0.8) (drill 0.4) (layers "F.Cu" "B.Cu") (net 3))
 (via (at 81.875695 39.350563) (size 0.8) (drill 0.4) (layers "F.Cu" "B.Cu") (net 3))
 (segment (start 77.970164 44.355542) (end 77.970164 43.927404) (width 0.25) (layer "B.Cu") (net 3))
 (segment (start 81.67131 39.350563) (end 81.875695 39.350563) (width 0.25) (layer "B.Cu") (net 3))
 (segment (start 77.970164 43.927404) (end 79.664848 42.23272) (width 0.25) (layer "B.Cu") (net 3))
 (segment (start 79.664848 42.23272) (end 81 40.897568) (width 0.25) (layer "B.Cu") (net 3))
 (segment (start 81 40.021873) (end 81.67131 39.350563) (width 0.25) (layer "B.Cu") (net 3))
 (segment (start 81 40.897568) (end 81 40.021873) (width 0.25) (layer "B.Cu") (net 3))
 (segment (start 81.517663 41.095969) (end 81.978632 40.635) (width 0.25) (layer "F.Cu") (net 4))
 (segment (start 81.517663 41.095969) (end 81.517663 42.192337) (width 0.25) (layer "F.Cu") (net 4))
 (segment (start 81.517663 42.192337) (end 80.99 42.72) (width 0.25) (layer "F.Cu") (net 4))
 (segment (start 81.978632 40.635) (end 82.6375 40.635) (width 0.25) (layer "F.Cu") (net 4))
 (segment (start 79.727599 43.274961) (end 80.435039 43.274961) (width 0.25) (layer "F.Cu") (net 4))
 (segment (start 80.435039 43.274961) (end 80.99 42.72) (width 0.25) (layer "F.Cu") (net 4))
 (via (at 80.99 42.72) (size 0.8) (drill 0.4) (layers "F.Cu" "B.Cu") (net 4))
 (segment (start 80.99 42.72) (end 78.796126 44.913874) (width 0.25) (layer "B.Cu") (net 4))
 (segment (start 78.796126 44.913874) (end 78.796126 45.704129) (width 0.25) (layer "B.Cu") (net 4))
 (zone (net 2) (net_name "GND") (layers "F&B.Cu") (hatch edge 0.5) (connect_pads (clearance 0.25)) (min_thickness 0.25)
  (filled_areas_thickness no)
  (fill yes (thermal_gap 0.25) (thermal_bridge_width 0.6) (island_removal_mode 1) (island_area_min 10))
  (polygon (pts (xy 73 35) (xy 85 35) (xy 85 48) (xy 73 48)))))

